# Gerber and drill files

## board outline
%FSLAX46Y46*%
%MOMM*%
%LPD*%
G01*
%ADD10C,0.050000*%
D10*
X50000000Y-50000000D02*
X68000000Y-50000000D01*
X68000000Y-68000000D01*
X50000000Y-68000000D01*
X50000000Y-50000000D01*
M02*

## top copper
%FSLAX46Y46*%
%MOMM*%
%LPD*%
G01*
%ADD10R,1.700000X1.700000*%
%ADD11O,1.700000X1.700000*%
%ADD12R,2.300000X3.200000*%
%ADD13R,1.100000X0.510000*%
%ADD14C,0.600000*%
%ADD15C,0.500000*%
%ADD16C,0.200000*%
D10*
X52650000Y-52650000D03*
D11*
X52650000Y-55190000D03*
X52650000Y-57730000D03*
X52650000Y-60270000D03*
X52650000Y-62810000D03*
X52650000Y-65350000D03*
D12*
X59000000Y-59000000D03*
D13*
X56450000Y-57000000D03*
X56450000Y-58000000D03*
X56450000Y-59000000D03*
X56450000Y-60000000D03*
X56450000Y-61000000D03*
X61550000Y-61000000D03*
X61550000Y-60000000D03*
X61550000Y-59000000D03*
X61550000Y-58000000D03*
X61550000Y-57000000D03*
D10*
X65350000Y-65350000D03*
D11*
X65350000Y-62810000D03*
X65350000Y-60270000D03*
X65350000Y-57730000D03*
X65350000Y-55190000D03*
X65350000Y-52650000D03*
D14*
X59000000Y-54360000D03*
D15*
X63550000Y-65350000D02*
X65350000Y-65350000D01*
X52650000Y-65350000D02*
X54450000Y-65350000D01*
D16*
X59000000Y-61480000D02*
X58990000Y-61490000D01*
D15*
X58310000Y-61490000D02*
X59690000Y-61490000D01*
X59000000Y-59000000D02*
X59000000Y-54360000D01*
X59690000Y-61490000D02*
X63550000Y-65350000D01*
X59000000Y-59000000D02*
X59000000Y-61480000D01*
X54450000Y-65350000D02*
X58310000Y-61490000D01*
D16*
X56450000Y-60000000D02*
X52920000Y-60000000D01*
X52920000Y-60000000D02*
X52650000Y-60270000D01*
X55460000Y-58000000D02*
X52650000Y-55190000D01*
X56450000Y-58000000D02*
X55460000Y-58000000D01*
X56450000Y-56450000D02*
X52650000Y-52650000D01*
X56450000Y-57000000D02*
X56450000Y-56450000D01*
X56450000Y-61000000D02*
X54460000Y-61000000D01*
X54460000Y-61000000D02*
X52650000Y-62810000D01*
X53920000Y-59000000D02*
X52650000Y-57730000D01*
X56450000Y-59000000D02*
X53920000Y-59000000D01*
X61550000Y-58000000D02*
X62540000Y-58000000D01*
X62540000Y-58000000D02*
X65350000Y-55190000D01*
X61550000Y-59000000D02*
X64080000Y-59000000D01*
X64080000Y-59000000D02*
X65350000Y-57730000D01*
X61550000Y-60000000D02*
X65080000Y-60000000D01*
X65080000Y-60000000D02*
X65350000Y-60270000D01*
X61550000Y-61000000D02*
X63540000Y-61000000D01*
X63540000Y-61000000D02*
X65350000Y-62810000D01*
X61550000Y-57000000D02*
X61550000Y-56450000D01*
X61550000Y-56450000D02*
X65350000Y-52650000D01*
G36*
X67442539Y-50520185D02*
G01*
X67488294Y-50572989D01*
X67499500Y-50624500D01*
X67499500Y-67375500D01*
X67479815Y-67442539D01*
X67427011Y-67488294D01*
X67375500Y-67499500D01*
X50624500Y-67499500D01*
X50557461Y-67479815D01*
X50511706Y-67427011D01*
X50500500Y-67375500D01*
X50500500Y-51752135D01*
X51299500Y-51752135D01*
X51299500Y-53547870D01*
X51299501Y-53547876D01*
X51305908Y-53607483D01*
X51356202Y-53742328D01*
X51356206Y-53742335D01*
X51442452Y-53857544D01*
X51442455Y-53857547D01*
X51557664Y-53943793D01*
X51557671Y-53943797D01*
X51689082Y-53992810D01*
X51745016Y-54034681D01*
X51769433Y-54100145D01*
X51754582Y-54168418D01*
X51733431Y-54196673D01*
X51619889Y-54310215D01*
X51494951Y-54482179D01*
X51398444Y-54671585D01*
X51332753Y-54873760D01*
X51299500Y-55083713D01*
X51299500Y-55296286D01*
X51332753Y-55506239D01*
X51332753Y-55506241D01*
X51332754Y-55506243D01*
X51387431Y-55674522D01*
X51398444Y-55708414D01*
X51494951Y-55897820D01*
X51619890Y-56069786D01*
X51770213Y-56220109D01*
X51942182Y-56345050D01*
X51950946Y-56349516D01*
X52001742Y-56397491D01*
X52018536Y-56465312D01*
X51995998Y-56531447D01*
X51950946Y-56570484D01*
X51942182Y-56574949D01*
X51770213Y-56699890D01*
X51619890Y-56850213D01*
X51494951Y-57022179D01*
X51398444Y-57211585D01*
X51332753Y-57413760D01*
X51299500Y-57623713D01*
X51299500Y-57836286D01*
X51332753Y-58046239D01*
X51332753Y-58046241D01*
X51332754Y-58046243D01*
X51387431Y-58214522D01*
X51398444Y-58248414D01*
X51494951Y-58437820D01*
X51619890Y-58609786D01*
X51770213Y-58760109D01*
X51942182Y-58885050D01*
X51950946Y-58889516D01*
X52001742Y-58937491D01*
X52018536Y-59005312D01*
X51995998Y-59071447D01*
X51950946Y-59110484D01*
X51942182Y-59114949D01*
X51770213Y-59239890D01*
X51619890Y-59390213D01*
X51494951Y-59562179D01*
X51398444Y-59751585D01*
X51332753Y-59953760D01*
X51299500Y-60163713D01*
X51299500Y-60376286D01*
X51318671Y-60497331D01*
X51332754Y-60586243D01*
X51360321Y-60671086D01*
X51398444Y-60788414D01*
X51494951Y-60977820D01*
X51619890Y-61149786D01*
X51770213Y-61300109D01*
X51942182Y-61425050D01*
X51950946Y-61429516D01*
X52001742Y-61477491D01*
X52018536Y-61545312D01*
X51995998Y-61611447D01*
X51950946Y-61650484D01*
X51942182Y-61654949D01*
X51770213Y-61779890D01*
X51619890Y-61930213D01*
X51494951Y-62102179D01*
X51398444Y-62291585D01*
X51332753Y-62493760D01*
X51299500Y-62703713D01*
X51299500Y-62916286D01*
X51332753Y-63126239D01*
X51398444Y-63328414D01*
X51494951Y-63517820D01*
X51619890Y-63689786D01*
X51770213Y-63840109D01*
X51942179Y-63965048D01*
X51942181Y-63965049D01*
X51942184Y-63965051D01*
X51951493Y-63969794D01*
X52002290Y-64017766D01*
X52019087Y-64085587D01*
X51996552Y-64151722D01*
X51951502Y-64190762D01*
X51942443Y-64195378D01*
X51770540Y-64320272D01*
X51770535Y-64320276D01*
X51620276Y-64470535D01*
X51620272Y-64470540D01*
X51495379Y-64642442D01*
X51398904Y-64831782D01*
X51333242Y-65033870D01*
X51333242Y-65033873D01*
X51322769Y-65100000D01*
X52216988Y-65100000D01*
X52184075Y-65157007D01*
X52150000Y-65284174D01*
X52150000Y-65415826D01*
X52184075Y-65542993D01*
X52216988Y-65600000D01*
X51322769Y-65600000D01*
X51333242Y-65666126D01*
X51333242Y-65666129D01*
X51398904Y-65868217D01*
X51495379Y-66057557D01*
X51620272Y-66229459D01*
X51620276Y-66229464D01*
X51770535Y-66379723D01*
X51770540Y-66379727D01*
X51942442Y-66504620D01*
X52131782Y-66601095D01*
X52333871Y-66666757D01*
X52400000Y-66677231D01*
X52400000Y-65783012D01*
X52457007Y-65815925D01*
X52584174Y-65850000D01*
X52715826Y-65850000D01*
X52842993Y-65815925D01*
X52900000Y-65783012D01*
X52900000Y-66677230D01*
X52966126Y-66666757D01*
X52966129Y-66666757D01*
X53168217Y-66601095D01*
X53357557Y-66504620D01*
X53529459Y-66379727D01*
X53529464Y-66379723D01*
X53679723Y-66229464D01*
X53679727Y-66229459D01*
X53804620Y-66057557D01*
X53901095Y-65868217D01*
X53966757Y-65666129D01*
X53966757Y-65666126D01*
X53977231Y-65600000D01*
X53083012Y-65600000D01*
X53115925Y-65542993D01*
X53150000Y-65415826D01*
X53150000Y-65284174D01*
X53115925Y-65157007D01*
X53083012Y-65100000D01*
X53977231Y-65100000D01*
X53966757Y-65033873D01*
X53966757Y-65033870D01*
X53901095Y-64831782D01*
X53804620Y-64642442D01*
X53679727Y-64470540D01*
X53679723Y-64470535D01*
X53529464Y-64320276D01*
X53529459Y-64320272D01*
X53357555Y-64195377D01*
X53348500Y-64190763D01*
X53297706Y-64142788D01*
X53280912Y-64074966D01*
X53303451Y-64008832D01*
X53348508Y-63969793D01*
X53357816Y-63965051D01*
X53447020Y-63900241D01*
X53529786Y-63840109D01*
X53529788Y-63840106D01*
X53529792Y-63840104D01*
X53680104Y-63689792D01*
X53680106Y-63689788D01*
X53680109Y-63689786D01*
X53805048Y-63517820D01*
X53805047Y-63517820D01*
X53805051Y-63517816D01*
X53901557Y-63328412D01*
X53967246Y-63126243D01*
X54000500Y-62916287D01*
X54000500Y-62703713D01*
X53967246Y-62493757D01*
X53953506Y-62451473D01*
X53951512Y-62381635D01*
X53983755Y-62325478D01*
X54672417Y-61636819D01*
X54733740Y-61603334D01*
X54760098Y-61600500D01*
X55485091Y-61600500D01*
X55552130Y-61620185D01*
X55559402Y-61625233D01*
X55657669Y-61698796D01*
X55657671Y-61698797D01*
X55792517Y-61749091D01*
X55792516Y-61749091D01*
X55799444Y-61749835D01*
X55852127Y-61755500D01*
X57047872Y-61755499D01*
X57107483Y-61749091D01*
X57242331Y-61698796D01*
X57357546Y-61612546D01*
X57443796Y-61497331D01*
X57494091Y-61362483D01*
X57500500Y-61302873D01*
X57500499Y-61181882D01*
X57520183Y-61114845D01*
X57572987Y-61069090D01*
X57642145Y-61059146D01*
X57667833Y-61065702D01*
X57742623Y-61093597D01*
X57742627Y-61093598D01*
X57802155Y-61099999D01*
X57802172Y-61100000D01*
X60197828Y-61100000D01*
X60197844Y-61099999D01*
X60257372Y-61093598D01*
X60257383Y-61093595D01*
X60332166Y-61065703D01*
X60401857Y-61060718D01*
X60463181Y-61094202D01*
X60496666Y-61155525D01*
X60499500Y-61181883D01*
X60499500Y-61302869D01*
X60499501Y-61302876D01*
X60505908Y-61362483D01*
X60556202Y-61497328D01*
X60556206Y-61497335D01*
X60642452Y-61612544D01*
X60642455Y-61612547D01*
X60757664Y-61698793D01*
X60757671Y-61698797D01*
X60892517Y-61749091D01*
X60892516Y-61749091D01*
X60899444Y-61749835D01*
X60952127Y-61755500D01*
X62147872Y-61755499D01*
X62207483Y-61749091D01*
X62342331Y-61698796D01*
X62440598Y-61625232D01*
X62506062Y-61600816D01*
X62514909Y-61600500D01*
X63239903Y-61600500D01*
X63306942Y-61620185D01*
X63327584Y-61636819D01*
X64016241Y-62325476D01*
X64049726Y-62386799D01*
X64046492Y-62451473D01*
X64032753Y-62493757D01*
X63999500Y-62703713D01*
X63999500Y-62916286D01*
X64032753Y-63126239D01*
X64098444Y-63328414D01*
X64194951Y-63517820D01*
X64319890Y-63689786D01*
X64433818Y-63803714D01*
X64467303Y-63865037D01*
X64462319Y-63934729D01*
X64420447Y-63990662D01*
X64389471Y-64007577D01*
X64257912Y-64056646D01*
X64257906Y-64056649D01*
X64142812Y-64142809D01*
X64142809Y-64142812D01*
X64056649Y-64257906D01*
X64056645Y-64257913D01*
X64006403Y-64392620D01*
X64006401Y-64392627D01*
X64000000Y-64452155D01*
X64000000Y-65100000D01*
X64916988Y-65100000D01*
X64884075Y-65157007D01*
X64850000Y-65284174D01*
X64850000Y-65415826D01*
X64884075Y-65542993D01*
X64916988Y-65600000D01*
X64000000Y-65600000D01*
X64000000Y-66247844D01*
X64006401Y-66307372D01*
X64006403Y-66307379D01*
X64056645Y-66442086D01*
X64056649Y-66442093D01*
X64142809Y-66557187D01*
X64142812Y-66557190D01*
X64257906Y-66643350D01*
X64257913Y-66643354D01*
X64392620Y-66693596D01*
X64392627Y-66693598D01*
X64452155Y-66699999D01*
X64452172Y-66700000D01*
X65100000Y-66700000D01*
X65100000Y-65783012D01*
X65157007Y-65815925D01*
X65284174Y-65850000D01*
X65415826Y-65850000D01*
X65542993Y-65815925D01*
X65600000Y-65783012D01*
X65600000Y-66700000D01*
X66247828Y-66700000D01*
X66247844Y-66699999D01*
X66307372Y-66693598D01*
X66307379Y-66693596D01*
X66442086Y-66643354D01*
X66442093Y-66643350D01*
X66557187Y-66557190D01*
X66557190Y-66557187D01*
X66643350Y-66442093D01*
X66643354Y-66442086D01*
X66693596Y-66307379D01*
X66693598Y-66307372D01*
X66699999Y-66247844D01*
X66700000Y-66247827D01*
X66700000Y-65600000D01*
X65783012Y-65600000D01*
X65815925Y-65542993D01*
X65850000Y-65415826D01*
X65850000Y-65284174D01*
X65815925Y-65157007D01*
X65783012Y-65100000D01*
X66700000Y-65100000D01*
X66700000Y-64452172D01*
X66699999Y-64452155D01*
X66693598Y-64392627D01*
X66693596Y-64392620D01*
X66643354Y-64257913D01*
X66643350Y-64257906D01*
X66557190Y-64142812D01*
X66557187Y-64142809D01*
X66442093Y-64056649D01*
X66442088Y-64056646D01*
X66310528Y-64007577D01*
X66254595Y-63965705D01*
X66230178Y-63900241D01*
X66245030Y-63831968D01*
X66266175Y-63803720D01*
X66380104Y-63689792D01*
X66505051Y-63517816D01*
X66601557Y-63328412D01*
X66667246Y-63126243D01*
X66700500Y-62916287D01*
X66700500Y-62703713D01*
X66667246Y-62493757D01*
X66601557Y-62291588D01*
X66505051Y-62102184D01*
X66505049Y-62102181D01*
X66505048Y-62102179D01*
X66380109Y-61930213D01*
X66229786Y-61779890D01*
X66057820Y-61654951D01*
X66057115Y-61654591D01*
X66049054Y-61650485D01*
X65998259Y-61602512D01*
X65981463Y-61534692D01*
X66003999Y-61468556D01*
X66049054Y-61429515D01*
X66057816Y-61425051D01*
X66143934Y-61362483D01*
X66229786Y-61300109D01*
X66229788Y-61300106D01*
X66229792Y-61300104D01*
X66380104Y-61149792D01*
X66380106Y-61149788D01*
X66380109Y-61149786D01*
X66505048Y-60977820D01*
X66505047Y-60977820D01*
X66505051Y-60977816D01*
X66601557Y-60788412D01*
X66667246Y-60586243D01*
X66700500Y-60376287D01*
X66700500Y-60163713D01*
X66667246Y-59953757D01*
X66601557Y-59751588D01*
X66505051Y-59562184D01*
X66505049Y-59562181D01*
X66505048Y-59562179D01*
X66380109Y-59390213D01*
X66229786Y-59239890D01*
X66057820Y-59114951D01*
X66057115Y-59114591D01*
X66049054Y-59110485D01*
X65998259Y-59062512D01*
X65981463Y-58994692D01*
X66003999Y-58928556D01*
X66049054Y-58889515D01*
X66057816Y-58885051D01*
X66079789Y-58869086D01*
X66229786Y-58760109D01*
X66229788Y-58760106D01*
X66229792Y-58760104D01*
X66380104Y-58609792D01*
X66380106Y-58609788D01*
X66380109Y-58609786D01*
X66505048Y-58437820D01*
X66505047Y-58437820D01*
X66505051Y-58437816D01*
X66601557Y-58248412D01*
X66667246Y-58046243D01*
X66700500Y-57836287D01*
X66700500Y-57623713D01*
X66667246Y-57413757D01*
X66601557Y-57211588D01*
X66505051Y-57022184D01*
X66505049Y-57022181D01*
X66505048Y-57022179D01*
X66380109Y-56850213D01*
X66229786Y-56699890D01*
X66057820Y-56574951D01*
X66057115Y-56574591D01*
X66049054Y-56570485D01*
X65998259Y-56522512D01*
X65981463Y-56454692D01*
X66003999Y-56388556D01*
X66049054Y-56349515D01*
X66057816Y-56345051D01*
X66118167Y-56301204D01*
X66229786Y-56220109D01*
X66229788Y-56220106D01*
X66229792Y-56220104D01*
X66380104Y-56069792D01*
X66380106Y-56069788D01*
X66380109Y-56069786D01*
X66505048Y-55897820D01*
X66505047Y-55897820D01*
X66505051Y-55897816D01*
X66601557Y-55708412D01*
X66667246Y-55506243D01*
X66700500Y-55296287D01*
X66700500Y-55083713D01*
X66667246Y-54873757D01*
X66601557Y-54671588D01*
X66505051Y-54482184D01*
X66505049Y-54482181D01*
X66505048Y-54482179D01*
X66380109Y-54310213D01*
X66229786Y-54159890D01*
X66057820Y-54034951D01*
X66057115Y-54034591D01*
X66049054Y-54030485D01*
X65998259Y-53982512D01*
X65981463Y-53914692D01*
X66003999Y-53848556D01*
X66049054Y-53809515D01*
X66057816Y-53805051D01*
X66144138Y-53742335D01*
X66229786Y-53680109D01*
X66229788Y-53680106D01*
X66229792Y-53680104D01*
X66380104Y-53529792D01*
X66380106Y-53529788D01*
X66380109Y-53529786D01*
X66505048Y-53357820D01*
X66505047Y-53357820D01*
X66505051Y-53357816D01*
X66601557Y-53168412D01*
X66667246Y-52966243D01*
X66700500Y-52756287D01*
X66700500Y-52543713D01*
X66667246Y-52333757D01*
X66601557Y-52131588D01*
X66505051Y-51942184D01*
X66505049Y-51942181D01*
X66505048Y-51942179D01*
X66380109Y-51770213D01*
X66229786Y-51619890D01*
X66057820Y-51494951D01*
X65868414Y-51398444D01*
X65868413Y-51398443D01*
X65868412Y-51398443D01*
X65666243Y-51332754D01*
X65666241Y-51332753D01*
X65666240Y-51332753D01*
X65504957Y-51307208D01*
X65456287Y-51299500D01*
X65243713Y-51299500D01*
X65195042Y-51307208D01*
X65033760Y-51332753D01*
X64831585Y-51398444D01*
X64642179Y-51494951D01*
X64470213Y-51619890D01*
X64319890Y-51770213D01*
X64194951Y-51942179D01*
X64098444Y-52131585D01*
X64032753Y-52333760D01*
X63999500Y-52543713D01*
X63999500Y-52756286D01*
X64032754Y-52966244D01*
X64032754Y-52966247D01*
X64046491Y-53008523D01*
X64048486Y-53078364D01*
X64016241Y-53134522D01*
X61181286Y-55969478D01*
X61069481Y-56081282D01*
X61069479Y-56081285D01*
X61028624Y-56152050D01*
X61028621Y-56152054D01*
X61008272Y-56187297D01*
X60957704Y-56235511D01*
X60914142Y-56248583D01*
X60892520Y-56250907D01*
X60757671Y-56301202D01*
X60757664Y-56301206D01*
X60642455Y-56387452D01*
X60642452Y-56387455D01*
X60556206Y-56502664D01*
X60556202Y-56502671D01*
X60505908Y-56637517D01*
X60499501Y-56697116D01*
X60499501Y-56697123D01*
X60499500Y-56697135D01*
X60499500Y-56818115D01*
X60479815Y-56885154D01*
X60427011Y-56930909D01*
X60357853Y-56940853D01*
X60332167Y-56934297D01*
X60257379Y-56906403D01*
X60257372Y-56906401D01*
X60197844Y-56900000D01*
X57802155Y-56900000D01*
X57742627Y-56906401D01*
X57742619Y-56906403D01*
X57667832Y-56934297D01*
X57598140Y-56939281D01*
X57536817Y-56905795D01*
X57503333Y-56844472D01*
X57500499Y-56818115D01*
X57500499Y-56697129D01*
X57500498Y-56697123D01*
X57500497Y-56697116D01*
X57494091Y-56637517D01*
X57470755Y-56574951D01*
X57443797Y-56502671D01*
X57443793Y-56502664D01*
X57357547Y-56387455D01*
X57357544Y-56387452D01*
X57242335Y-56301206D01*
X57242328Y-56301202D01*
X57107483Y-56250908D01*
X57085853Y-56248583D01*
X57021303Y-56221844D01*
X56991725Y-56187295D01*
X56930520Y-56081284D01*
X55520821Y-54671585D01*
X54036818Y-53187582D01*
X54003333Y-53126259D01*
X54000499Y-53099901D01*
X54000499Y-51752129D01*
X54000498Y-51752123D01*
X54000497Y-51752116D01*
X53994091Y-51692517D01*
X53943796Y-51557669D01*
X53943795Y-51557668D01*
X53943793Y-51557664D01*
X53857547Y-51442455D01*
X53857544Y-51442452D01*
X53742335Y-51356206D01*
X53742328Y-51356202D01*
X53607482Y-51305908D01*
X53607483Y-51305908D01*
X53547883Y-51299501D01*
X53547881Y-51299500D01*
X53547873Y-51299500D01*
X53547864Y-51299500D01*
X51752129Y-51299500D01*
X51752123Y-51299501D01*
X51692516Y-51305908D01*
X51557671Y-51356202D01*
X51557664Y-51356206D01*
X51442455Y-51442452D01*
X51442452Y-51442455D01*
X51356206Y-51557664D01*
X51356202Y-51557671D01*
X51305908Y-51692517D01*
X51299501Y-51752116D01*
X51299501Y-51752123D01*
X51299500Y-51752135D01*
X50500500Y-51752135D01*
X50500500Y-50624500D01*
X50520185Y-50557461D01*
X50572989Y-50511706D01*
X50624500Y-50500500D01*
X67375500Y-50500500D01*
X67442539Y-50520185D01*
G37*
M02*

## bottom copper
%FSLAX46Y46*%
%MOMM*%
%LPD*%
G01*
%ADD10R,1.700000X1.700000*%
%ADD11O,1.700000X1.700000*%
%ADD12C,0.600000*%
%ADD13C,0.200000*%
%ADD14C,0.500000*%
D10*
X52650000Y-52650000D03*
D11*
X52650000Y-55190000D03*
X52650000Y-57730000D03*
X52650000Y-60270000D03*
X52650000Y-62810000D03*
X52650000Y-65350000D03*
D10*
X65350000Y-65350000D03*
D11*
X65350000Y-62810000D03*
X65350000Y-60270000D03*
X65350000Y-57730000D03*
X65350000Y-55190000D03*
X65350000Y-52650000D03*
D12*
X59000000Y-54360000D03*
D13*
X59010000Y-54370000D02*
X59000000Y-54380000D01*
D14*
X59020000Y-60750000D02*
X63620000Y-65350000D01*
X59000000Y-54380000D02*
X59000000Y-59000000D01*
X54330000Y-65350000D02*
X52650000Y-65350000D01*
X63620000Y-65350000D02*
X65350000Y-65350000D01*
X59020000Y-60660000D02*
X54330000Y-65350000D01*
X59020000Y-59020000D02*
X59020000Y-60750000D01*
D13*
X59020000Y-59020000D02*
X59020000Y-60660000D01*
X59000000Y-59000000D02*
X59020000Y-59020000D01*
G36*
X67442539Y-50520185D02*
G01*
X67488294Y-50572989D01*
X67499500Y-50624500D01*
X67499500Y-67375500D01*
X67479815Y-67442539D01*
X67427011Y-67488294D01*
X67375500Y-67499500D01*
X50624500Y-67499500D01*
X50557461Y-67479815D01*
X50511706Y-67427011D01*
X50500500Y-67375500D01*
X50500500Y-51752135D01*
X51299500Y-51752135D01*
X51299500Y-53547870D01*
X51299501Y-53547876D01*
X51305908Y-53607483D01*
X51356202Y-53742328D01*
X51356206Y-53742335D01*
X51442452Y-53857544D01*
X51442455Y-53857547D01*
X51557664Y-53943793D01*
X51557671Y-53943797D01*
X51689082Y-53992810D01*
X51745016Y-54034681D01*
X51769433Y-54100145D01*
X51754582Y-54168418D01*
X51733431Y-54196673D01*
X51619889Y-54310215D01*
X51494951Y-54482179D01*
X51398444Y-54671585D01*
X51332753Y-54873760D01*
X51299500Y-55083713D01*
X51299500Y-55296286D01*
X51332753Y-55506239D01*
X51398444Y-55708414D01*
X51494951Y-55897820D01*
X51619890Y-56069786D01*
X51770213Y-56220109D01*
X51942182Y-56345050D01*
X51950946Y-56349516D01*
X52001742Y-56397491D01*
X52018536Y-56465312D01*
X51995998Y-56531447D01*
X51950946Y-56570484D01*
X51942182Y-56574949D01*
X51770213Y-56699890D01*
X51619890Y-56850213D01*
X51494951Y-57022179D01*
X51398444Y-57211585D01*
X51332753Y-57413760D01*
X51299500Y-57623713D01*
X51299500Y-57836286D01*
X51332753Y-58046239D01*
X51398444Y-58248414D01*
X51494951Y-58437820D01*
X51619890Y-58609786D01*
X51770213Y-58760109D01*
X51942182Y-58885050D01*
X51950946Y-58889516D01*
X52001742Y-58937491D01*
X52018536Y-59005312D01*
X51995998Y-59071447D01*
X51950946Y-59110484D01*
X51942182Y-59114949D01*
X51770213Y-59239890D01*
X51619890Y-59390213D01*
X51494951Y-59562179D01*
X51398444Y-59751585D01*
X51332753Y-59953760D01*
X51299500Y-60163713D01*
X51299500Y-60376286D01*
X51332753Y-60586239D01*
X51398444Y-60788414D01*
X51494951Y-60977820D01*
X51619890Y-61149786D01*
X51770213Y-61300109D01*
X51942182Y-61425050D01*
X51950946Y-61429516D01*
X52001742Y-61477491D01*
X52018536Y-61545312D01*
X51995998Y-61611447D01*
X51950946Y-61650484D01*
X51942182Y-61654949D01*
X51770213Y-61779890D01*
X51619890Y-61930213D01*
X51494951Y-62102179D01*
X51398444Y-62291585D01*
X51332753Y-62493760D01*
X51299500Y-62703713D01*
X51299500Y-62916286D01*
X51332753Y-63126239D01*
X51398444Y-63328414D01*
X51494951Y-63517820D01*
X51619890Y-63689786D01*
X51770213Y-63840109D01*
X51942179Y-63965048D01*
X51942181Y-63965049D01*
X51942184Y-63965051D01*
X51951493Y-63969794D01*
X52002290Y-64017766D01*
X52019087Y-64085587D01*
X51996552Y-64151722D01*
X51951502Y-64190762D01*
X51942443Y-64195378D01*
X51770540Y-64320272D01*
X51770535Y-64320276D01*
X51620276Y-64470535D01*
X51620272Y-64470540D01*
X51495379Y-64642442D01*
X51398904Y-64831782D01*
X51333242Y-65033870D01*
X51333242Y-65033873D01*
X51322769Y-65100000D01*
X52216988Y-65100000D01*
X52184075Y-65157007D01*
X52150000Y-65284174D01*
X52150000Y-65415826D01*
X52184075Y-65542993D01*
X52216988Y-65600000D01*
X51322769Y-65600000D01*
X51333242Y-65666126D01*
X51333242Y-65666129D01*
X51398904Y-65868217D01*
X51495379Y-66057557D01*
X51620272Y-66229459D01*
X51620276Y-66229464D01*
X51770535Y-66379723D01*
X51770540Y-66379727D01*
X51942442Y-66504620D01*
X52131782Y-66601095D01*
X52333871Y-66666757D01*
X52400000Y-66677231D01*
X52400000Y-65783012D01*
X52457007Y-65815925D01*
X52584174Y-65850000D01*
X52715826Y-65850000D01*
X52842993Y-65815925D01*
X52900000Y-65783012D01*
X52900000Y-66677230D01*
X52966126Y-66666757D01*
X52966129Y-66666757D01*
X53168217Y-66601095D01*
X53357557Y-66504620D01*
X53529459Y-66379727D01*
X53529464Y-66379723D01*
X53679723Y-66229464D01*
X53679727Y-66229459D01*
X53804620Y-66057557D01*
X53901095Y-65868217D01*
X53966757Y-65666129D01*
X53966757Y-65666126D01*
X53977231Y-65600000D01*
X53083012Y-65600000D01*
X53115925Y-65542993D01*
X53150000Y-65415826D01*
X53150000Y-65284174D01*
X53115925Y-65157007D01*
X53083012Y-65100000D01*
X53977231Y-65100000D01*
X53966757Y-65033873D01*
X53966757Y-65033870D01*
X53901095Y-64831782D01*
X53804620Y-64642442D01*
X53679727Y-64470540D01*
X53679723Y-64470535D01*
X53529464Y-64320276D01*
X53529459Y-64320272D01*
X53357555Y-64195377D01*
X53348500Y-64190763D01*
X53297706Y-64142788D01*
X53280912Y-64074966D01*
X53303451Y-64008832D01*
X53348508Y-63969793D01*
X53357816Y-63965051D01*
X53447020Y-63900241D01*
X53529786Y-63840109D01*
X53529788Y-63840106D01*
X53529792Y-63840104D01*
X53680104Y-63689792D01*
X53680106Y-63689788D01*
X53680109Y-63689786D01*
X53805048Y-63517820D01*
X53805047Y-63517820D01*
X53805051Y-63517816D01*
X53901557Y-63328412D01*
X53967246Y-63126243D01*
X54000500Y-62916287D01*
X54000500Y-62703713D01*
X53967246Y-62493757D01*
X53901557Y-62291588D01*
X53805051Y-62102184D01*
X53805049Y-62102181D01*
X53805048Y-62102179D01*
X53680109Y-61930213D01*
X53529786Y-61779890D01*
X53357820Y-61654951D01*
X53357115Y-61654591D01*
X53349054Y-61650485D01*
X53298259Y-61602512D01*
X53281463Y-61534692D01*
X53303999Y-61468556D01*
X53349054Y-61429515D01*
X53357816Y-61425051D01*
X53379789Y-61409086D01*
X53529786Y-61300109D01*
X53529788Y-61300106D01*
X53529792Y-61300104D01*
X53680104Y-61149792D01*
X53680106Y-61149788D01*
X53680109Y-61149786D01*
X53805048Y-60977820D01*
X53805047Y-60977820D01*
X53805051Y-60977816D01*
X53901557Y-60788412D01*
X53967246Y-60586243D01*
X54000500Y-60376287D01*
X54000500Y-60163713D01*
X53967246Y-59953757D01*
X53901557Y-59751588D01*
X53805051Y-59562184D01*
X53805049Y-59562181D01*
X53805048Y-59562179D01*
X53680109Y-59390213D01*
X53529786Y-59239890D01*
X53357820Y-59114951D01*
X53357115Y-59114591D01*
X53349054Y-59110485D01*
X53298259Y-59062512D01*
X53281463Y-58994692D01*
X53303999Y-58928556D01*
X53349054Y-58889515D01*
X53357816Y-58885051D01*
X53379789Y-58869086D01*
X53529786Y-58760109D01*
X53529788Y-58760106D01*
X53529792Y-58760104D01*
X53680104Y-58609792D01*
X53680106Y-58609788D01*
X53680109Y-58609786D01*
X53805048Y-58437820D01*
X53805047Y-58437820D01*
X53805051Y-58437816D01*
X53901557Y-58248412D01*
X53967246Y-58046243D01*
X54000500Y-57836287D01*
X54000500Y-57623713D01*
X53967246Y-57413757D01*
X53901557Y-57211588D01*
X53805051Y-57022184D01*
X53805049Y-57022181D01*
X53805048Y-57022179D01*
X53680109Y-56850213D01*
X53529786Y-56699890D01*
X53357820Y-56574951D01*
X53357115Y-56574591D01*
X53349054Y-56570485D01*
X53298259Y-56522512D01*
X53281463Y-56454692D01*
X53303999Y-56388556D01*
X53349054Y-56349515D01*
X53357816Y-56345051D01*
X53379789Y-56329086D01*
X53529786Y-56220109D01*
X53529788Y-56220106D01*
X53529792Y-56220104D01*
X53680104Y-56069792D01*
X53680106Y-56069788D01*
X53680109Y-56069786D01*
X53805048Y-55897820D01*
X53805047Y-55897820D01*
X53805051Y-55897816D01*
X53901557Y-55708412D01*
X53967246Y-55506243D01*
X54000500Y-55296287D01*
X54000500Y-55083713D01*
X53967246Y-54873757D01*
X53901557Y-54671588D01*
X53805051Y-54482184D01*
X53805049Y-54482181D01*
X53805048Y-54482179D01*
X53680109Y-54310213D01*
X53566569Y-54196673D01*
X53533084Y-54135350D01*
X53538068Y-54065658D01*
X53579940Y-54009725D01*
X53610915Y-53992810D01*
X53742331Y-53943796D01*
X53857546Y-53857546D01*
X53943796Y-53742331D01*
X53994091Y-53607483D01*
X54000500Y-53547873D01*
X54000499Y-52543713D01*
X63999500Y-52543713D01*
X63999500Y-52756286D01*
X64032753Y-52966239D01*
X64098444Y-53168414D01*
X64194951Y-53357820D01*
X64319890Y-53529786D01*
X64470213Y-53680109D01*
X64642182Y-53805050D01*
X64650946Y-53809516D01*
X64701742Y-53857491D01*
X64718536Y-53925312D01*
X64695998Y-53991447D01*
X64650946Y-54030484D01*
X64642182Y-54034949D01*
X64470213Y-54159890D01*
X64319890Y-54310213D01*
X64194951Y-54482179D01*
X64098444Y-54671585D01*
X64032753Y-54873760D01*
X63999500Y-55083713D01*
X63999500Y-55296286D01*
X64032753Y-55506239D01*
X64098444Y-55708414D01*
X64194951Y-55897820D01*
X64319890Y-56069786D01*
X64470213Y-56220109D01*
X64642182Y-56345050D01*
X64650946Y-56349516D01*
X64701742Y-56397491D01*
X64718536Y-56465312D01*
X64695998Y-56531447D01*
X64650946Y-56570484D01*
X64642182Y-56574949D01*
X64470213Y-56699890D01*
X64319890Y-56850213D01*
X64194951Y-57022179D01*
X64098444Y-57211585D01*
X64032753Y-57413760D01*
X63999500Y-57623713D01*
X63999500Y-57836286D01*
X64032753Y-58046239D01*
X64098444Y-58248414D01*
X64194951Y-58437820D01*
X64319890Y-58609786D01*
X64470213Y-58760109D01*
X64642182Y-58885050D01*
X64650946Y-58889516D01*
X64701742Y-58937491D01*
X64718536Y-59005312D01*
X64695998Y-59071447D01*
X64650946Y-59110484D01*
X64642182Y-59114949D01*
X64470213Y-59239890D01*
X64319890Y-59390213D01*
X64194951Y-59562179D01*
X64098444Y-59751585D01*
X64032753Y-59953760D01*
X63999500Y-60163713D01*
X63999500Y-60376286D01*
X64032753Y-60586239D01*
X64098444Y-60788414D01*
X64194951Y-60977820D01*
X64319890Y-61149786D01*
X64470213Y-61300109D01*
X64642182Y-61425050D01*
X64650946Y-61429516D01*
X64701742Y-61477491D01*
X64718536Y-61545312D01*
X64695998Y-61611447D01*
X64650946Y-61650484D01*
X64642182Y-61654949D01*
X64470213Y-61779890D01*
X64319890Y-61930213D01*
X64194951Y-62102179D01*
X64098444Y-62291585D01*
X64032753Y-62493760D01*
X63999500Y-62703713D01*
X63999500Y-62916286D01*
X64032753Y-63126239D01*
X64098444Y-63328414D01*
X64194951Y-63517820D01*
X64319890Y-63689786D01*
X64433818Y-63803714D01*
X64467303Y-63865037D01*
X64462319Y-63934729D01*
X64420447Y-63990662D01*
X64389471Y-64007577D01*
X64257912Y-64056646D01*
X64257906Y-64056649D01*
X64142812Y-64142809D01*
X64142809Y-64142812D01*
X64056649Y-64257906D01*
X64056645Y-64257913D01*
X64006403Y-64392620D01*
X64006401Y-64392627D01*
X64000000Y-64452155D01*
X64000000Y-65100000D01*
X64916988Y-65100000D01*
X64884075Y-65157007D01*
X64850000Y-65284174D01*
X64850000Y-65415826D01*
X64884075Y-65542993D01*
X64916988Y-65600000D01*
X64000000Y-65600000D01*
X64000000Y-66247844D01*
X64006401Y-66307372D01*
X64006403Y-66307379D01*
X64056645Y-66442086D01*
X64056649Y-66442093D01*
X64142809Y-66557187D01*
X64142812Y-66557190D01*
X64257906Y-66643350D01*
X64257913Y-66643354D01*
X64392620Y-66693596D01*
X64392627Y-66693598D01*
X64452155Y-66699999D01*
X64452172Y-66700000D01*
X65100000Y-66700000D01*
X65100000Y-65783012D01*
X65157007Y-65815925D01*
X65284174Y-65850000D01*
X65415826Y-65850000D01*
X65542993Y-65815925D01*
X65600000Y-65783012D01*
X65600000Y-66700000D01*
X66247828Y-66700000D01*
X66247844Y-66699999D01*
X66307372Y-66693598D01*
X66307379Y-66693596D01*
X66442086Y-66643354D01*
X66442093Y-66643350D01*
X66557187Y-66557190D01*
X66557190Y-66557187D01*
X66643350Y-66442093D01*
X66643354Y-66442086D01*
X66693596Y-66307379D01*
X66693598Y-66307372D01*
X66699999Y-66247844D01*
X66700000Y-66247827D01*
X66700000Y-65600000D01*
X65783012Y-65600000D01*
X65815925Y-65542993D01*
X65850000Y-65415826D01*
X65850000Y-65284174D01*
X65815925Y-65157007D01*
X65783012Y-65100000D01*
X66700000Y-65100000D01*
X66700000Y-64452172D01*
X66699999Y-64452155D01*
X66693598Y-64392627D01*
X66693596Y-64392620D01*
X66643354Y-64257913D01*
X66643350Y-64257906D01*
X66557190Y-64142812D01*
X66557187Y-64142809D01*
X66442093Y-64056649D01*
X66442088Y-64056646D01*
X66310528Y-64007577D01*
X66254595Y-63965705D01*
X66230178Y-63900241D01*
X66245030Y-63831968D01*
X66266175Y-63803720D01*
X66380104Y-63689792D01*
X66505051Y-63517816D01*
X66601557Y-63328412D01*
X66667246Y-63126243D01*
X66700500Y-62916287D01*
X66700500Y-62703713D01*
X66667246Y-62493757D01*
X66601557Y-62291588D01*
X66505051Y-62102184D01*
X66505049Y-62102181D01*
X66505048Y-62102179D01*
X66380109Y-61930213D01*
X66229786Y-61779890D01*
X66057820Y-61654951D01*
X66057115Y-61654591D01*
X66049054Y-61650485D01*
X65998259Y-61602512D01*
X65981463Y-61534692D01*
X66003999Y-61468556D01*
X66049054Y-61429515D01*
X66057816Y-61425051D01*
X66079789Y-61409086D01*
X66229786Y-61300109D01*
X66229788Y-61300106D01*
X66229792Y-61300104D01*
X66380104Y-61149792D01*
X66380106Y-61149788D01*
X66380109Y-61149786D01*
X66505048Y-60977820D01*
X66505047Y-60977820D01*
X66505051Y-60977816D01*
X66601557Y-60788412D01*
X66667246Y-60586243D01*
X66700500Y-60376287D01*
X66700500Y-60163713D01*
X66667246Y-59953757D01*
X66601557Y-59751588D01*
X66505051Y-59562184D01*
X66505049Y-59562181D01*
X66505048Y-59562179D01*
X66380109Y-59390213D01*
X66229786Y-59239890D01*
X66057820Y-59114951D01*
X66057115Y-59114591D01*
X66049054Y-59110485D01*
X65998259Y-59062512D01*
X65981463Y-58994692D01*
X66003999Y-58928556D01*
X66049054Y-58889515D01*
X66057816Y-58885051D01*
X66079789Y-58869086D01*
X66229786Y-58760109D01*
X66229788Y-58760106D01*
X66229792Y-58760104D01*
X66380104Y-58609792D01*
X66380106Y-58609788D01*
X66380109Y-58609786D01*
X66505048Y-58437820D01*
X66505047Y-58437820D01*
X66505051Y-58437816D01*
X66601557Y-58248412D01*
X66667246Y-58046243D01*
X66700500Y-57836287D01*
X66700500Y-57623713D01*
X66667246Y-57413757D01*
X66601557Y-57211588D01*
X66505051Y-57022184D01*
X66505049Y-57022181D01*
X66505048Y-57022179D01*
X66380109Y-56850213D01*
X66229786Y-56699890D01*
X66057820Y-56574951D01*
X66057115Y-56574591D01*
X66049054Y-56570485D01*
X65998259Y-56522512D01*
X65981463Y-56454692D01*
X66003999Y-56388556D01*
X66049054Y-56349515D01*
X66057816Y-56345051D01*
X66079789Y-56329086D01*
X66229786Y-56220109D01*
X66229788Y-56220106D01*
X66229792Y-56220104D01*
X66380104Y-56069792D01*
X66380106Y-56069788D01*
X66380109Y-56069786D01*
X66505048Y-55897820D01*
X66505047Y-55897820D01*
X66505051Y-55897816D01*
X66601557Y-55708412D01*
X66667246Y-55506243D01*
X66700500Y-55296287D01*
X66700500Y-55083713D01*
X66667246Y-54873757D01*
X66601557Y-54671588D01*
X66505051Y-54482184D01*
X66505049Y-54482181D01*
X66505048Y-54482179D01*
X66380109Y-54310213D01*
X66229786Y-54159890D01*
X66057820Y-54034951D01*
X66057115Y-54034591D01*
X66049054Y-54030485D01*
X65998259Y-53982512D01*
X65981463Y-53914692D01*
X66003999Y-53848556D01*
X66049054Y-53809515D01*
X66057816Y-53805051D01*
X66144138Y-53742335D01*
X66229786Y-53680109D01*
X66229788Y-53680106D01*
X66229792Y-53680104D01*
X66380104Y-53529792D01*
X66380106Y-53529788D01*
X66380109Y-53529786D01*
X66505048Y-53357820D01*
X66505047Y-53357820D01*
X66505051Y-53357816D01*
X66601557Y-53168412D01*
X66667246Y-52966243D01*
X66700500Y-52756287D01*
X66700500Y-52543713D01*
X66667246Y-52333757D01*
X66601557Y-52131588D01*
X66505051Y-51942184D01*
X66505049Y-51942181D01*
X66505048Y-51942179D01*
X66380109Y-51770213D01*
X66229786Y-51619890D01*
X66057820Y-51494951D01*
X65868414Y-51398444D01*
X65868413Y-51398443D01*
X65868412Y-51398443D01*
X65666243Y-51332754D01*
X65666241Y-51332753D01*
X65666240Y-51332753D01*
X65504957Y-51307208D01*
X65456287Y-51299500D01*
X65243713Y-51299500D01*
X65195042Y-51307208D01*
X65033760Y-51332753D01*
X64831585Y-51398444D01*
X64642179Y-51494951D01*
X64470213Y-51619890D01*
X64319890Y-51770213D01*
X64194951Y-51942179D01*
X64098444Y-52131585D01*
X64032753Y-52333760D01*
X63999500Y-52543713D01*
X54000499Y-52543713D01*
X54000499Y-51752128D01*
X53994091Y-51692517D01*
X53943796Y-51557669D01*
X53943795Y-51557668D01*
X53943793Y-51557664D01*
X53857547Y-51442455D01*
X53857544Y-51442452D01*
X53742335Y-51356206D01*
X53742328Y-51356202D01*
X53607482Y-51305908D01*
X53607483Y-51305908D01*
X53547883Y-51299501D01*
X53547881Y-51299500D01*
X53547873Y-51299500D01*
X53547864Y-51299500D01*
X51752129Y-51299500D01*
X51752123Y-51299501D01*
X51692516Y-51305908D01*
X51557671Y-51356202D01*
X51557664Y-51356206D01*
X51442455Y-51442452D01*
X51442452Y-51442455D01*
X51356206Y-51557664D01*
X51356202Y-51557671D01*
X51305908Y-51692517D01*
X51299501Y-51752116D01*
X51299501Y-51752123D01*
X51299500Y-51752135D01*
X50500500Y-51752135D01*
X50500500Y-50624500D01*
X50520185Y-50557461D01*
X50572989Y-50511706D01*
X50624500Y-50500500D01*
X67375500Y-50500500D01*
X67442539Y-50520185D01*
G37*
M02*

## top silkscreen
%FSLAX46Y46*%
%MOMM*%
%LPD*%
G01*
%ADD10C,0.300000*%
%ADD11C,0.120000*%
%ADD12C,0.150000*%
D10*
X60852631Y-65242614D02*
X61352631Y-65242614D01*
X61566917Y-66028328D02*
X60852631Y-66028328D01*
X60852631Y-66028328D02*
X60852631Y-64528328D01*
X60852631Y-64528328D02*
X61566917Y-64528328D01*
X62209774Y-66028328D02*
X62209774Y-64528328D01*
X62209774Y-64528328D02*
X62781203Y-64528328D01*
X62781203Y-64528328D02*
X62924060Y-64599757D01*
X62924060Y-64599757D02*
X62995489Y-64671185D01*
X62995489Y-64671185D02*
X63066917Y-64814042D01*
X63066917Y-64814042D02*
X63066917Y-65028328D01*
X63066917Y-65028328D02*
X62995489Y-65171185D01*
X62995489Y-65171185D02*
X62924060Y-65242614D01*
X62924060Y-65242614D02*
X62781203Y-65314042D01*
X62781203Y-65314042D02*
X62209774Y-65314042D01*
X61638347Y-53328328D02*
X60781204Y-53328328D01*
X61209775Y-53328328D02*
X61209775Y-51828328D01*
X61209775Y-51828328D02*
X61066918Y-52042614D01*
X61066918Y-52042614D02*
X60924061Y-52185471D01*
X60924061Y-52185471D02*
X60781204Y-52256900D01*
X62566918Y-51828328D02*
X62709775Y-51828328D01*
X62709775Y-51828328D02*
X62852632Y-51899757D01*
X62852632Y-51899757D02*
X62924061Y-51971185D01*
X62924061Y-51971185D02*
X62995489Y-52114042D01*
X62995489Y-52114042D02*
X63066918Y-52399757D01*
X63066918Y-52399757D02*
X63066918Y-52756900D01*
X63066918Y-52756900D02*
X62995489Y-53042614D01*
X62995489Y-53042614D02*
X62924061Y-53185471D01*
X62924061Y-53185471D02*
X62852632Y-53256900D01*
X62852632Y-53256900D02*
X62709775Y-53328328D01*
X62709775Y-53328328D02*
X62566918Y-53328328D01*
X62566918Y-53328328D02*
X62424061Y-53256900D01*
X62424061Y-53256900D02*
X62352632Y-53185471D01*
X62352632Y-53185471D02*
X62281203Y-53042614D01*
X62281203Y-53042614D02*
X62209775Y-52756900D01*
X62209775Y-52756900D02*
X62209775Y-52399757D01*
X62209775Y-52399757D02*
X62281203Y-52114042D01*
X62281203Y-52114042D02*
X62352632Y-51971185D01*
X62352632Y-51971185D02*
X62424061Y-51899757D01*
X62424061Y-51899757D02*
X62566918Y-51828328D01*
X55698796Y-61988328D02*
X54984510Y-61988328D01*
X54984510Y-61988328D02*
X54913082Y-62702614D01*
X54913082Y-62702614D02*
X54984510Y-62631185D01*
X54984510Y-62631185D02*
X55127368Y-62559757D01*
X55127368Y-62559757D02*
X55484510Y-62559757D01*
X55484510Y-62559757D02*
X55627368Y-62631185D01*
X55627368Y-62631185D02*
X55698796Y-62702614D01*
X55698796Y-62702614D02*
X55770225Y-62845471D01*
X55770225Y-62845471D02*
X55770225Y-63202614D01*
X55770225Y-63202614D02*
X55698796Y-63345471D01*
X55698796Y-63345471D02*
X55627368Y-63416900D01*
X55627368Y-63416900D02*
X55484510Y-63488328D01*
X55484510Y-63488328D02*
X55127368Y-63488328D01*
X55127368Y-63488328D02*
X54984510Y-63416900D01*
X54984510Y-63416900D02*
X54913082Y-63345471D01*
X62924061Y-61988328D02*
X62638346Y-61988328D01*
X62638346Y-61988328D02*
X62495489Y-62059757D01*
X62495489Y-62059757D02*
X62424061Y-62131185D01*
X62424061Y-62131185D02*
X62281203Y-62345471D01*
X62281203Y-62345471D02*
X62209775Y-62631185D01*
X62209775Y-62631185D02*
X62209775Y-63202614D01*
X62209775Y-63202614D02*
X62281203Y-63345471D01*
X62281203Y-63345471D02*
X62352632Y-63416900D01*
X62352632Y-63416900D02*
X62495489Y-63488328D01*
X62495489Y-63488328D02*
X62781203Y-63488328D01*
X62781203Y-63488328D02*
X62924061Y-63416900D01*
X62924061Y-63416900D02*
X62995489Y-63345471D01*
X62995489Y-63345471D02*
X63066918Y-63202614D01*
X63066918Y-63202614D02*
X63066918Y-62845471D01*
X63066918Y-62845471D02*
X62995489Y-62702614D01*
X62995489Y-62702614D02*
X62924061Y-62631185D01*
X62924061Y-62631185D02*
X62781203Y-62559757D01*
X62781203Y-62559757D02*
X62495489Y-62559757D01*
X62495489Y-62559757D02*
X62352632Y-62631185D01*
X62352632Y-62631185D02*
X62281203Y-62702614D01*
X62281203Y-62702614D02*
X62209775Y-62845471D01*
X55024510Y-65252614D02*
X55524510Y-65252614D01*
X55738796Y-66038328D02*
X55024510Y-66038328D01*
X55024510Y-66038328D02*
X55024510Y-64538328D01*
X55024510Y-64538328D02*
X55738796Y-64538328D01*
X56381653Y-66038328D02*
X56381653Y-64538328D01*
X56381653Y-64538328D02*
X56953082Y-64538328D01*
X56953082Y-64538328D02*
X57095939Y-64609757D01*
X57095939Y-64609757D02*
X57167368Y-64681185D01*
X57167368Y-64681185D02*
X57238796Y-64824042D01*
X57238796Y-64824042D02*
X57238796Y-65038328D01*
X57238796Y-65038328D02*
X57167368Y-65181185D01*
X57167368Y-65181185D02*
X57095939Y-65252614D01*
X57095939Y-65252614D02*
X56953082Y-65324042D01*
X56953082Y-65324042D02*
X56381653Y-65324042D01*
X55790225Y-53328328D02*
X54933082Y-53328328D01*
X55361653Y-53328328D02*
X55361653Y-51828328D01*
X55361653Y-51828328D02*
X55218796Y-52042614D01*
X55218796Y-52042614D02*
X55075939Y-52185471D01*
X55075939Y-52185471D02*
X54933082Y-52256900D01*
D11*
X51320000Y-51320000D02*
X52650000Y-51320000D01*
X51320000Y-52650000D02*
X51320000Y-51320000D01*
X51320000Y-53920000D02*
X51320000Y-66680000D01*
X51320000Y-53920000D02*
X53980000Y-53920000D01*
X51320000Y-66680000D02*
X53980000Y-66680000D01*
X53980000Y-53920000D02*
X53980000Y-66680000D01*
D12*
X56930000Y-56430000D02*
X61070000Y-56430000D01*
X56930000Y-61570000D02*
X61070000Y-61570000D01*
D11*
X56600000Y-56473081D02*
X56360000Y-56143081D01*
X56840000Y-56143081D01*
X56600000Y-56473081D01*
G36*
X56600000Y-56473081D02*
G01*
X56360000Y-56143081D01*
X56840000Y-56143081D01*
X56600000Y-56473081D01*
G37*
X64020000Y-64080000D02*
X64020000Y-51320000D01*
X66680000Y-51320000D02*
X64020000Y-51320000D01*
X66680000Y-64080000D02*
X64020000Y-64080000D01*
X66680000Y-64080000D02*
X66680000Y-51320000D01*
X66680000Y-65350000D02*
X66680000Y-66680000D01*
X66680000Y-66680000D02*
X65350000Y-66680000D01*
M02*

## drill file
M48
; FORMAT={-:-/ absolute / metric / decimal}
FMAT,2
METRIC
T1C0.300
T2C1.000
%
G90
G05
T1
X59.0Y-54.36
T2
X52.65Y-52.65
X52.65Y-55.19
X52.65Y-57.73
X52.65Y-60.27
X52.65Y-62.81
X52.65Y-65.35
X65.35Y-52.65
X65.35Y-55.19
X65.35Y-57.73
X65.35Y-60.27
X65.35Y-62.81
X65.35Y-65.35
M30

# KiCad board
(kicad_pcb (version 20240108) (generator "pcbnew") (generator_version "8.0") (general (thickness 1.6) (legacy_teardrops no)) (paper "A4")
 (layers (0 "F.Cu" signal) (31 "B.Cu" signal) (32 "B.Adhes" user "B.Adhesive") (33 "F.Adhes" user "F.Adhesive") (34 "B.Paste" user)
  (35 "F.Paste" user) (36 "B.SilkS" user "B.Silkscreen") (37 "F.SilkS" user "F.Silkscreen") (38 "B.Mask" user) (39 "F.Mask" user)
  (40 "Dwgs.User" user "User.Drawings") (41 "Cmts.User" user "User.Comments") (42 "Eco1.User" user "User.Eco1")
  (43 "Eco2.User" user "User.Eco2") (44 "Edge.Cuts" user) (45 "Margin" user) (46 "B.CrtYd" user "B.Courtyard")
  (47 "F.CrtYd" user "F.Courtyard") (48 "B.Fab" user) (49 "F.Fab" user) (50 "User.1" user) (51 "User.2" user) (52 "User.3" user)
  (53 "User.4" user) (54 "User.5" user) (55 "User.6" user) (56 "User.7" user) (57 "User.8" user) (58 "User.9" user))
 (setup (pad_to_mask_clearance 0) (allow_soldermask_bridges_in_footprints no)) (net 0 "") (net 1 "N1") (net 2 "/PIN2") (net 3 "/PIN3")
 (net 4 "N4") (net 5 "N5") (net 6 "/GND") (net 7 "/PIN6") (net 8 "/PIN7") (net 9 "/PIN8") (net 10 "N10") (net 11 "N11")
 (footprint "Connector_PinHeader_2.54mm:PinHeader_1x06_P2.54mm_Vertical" (layer "F.Cu") (at 52.65 52.65)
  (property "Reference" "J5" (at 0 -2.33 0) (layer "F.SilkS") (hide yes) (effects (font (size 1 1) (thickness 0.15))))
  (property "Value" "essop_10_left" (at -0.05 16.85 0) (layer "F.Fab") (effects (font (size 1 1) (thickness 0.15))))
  (fp_line (start -1.33 -1.33) (end 0 -1.33) (stroke (width 0.12) (type solid)) (layer "F.SilkS"))
  (fp_line (start -1.33 0) (end -1.33 -1.33) (stroke (width 0.12) (type solid)) (layer "F.SilkS"))
  (fp_line (start -1.33 1.27) (end -1.33 14.03) (stroke (width 0.12) (type solid)) (layer "F.SilkS"))
  (fp_line (start -1.33 1.27) (end 1.33 1.27) (stroke (width 0.12) (type solid)) (layer "F.SilkS"))
  (fp_line (start -1.33 14.03) (end 1.33 14.03) (stroke (width 0.12) (type solid)) (layer "F.SilkS"))
  (fp_line (start 1.33 1.27) (end 1.33 14.03) (stroke (width 0.12) (type solid)) (layer "F.SilkS"))
  (pad "1" thru_hole rect (at 0 0) (size 1.7 1.7) (drill 1) (layers "*.Cu" "*.Mask") (remove_unused_layers no) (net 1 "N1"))
  (pad "2" thru_hole oval (at 0 2.54) (size 1.7 1.7) (drill 1) (layers "*.Cu" "*.Mask") (remove_unused_layers no) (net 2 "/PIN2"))
  (pad "3" thru_hole oval (at 0 5.08) (size 1.7 1.7) (drill 1) (layers "*.Cu" "*.Mask") (remove_unused_layers no) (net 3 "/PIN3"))
  (pad "4" thru_hole oval (at 0 7.62) (size 1.7 1.7) (drill 1) (layers "*.Cu" "*.Mask") (remove_unused_layers no) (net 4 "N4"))
  (pad "5" thru_hole oval (at 0 10.16) (size 1.7 1.7) (drill 1) (layers "*.Cu" "*.Mask") (remove_unused_layers no) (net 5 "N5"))
  (pad "6" thru_hole oval (at 0 12.7) (size 1.7 1.7) (drill 1) (layers "*.Cu" "*.Mask") (remove_unused_layers no) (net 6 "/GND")))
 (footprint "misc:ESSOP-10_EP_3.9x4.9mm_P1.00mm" (layer "F.Cu") (at 59 59)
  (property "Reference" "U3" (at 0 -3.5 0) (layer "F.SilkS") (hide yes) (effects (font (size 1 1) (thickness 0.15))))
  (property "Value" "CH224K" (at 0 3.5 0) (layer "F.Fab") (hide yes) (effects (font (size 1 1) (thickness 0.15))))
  (fp_line (start -2.07 -2.57) (end 2.07 -2.57) (stroke (width 0.15) (type solid)) (layer "F.SilkS"))
  (fp_line (start -2.07 2.57) (end 2.07 2.57) (stroke (width 0.15) (type solid)) (layer "F.SilkS"))
  (fp_poly
   (pts (xy -2.4 -2.526919) (xy -2.64 -2.856919) (xy -2.16 -2.856919) (xy -2.4 -2.526919)) (stroke (width 0.12) (type solid)) (fill solid)
   (layer "F.SilkS"))
  (pad "0" smd rect (at 0 0 90) (size 3.2 2.3) (layers "F.Cu" "F.Paste" "F.Mask") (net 6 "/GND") (thermal_bridge_angle 45))
  (pad "1" smd rect (at -2.55 -2) (size 1.1 0.51) (layers "F.Cu" "F.Paste" "F.Mask") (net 1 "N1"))
  (pad "2" smd rect (at -2.55 -1) (size 1.1 0.51) (layers "F.Cu" "F.Paste" "F.Mask") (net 2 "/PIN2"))
  (pad "3" smd rect (at -2.55 0) (size 1.1 0.51) (layers "F.Cu" "F.Paste" "F.Mask") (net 3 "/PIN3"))
  (pad "4" smd rect (at -2.55 1) (size 1.1 0.51) (layers "F.Cu" "F.Paste" "F.Mask") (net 4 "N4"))
  (pad "5" smd rect (at -2.55 2) (size 1.1 0.51) (layers "F.Cu" "F.Paste" "F.Mask") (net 5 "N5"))
  (pad "6" smd rect (at 2.55 2) (size 1.1 0.51) (layers "F.Cu" "F.Paste" "F.Mask") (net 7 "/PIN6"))
  (pad "7" smd rect (at 2.55 1) (size 1.1 0.51) (layers "F.Cu" "F.Paste" "F.Mask") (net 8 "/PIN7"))
  (pad "8" smd rect (at 2.55 0) (size 1.1 0.51) (layers "F.Cu" "F.Paste" "F.Mask") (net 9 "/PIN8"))
  (pad "9" smd rect (at 2.55 -1) (size 1.1 0.51) (layers "F.Cu" "F.Paste" "F.Mask") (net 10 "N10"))
  (pad "10" smd rect (at 2.55 -2) (size 1.1 0.51) (layers "F.Cu" "F.Paste" "F.Mask") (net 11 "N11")))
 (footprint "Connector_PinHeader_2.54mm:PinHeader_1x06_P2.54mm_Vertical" (layer "F.Cu") (at 65.35 65.35 180)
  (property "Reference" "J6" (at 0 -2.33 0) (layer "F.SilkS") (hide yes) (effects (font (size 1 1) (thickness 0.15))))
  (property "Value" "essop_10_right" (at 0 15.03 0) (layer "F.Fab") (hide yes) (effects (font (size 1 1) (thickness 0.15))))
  (fp_line (start 1.33 1.27) (end 1.33 14.03) (stroke (width 0.12) (type solid)) (layer "F.SilkS"))
  (fp_line (start -1.33 14.03) (end 1.33 14.03) (stroke (width 0.12) (type solid)) (layer "F.SilkS"))
  (fp_line (start -1.33 1.27) (end 1.33 1.27) (stroke (width 0.12) (type solid)) (layer "F.SilkS"))
  (fp_line (start -1.33 1.27) (end -1.33 14.03) (stroke (width 0.12) (type solid)) (layer "F.SilkS"))
  (fp_line (start -1.33 0) (end -1.33 -1.33) (stroke (width 0.12) (type solid)) (layer "F.SilkS"))
  (fp_line (start -1.33 -1.33) (end 0 -1.33) (stroke (width 0.12) (type solid)) (layer "F.SilkS"))
  (pad "1" thru_hole rect (at 0 0 180) (size 1.7 1.7) (drill 1) (layers "*.Cu" "*.Mask") (remove_unused_layers no) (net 6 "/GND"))
  (pad "2" thru_hole oval (at 0 2.54 180) (size 1.7 1.7) (drill 1) (layers "*.Cu" "*.Mask") (remove_unused_layers no) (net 7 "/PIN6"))
  (pad "3" thru_hole oval (at 0 5.08 180) (size 1.7 1.7) (drill 1) (layers "*.Cu" "*.Mask") (remove_unused_layers no) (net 8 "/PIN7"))
  (pad "4" thru_hole oval (at 0 7.62 180) (size 1.7 1.7) (drill 1) (layers "*.Cu" "*.Mask") (remove_unused_layers no) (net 9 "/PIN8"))
  (pad "5" thru_hole oval (at 0 10.16 180) (size 1.7 1.7) (drill 1) (layers "*.Cu" "*.Mask") (remove_unused_layers no) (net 10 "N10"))
  (pad "6" thru_hole oval (at 0 12.7 180) (size 1.7 1.7) (drill 1) (layers "*.Cu" "*.Mask") (remove_unused_layers no) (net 11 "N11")))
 (gr_rect (start 50 50) (end 68 68) (stroke (width 0.05) (type default)) (fill none) (layer "Edge.Cuts"))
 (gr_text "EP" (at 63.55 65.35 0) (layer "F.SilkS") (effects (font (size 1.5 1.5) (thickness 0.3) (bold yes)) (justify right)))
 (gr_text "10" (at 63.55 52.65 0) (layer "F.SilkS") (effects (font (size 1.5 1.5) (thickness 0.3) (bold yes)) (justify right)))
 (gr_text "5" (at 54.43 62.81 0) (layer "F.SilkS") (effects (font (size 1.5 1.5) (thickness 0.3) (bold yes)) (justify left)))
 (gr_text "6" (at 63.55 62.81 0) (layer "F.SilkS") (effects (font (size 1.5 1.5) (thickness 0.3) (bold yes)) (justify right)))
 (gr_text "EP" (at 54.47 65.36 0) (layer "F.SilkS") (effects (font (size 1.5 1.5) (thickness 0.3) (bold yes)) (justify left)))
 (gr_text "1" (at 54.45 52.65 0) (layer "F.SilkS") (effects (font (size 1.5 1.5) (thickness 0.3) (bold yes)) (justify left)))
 (segment (start 63.55 65.35) (end 65.35 65.35) (width 0.5) (layer "F.Cu") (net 6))
 (segment (start 52.65 65.35) (end 54.45 65.35) (width 0.5) (layer "F.Cu") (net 6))
 (segment (start 59 61.48) (end 58.99 61.49) (width 0.2) (layer "F.Cu") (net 6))
 (segment (start 58.31 61.49) (end 59.69 61.49) (width 0.5) (layer "F.Cu") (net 6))
 (segment (start 59 59) (end 59 54.36) (width 0.5) (layer "F.Cu") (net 6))
 (segment (start 59.69 61.49) (end 63.55 65.35) (width 0.5) (layer "F.Cu") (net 6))
 (segment (start 59 59) (end 59 61.48) (width 0.5) (layer "F.Cu") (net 6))
 (segment (start 54.45 65.35) (end 58.31 61.49) (width 0.5) (layer "F.Cu") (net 6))
 (via (at 59 54.36) (size 0.6) (drill 0.3) (layers "F.Cu" "B.Cu") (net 6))
 (segment (start 59.01 54.37) (end 59 54.38) (width 0.2) (layer "B.Cu") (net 6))
 (segment (start 59.02 60.75) (end 63.62 65.35) (width 0.5) (layer "B.Cu") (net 6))
 (segment (start 59 54.38) (end 59 59) (width 0.5) (layer "B.Cu") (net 6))
 (segment (start 54.33 65.35) (end 52.65 65.35) (width 0.5) (layer "B.Cu") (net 6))
 (segment (start 63.62 65.35) (end 65.35 65.35) (width 0.5) (layer "B.Cu") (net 6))
 (segment (start 59.02 60.66) (end 54.33 65.35) (width 0.5) (layer "B.Cu") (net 6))
 (segment (start 59.02 59.02) (end 59.02 60.75) (width 0.5) (layer "B.Cu") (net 6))
 (segment (start 59.02 59.02) (end 59.02 60.66) (width 0.2) (layer "B.Cu") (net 6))
 (segment (start 59 59) (end 59.02 59.02) (width 0.2) (layer "B.Cu") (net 6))
 (segment (start 56.45 60) (end 52.92 60) (width 0.2) (layer "F.Cu") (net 4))
 (segment (start 52.92 60) (end 52.65 60.27) (width 0.2) (layer "F.Cu") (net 4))
 (segment (start 55.46 58) (end 52.65 55.19) (width 0.2) (layer "F.Cu") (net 2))
 (segment (start 56.45 58) (end 55.46 58) (width 0.2) (layer "F.Cu") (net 2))
 (segment (start 56.45 56.45) (end 52.65 52.65) (width 0.2) (layer "F.Cu") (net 1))
 (segment (start 56.45 57) (end 56.45 56.45) (width 0.2) (layer "F.Cu") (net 1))
 (segment (start 56.45 61) (end 54.46 61) (width 0.2) (layer "F.Cu") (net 5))
 (segment (start 54.46 61) (end 52.65 62.81) (width 0.2) (layer "F.Cu") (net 5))
 (segment (start 53.92 59) (end 52.65 57.73) (width 0.2) (layer "F.Cu") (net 3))
 (segment (start 56.45 59) (end 53.92 59) (width 0.2) (layer "F.Cu") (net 3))
 (segment (start 61.55 58) (end 62.54 58) (width 0.2) (layer "F.Cu") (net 10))
 (segment (start 62.54 58) (end 65.35 55.19) (width 0.2) (layer "F.Cu") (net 10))
 (segment (start 61.55 59) (end 64.08 59) (width 0.2) (layer "F.Cu") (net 9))
 (segment (start 64.08 59) (end 65.35 57.73) (width 0.2) (layer "F.Cu") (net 9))
 (segment (start 61.55 60) (end 65.08 60) (width 0.2) (layer "F.Cu") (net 8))
 (segment (start 65.08 60) (end 65.35 60.27) (width 0.2) (layer "F.Cu") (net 8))
 (segment (start 61.55 61) (end 63.54 61) (width 0.2) (layer "F.Cu") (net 7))
 (segment (start 63.54 61) (end 65.35 62.81) (width 0.2) (layer "F.Cu") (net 7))
 (segment (start 61.55 57) (end 61.55 56.45) (width 0.2) (layer "F.Cu") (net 11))
 (segment (start 61.55 56.45) (end 65.35 52.65) (width 0.2) (layer "F.Cu") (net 11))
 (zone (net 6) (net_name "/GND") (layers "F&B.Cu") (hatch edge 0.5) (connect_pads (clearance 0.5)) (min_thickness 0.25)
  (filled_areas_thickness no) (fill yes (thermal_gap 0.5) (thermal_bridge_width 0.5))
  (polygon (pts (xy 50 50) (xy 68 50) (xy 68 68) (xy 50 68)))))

